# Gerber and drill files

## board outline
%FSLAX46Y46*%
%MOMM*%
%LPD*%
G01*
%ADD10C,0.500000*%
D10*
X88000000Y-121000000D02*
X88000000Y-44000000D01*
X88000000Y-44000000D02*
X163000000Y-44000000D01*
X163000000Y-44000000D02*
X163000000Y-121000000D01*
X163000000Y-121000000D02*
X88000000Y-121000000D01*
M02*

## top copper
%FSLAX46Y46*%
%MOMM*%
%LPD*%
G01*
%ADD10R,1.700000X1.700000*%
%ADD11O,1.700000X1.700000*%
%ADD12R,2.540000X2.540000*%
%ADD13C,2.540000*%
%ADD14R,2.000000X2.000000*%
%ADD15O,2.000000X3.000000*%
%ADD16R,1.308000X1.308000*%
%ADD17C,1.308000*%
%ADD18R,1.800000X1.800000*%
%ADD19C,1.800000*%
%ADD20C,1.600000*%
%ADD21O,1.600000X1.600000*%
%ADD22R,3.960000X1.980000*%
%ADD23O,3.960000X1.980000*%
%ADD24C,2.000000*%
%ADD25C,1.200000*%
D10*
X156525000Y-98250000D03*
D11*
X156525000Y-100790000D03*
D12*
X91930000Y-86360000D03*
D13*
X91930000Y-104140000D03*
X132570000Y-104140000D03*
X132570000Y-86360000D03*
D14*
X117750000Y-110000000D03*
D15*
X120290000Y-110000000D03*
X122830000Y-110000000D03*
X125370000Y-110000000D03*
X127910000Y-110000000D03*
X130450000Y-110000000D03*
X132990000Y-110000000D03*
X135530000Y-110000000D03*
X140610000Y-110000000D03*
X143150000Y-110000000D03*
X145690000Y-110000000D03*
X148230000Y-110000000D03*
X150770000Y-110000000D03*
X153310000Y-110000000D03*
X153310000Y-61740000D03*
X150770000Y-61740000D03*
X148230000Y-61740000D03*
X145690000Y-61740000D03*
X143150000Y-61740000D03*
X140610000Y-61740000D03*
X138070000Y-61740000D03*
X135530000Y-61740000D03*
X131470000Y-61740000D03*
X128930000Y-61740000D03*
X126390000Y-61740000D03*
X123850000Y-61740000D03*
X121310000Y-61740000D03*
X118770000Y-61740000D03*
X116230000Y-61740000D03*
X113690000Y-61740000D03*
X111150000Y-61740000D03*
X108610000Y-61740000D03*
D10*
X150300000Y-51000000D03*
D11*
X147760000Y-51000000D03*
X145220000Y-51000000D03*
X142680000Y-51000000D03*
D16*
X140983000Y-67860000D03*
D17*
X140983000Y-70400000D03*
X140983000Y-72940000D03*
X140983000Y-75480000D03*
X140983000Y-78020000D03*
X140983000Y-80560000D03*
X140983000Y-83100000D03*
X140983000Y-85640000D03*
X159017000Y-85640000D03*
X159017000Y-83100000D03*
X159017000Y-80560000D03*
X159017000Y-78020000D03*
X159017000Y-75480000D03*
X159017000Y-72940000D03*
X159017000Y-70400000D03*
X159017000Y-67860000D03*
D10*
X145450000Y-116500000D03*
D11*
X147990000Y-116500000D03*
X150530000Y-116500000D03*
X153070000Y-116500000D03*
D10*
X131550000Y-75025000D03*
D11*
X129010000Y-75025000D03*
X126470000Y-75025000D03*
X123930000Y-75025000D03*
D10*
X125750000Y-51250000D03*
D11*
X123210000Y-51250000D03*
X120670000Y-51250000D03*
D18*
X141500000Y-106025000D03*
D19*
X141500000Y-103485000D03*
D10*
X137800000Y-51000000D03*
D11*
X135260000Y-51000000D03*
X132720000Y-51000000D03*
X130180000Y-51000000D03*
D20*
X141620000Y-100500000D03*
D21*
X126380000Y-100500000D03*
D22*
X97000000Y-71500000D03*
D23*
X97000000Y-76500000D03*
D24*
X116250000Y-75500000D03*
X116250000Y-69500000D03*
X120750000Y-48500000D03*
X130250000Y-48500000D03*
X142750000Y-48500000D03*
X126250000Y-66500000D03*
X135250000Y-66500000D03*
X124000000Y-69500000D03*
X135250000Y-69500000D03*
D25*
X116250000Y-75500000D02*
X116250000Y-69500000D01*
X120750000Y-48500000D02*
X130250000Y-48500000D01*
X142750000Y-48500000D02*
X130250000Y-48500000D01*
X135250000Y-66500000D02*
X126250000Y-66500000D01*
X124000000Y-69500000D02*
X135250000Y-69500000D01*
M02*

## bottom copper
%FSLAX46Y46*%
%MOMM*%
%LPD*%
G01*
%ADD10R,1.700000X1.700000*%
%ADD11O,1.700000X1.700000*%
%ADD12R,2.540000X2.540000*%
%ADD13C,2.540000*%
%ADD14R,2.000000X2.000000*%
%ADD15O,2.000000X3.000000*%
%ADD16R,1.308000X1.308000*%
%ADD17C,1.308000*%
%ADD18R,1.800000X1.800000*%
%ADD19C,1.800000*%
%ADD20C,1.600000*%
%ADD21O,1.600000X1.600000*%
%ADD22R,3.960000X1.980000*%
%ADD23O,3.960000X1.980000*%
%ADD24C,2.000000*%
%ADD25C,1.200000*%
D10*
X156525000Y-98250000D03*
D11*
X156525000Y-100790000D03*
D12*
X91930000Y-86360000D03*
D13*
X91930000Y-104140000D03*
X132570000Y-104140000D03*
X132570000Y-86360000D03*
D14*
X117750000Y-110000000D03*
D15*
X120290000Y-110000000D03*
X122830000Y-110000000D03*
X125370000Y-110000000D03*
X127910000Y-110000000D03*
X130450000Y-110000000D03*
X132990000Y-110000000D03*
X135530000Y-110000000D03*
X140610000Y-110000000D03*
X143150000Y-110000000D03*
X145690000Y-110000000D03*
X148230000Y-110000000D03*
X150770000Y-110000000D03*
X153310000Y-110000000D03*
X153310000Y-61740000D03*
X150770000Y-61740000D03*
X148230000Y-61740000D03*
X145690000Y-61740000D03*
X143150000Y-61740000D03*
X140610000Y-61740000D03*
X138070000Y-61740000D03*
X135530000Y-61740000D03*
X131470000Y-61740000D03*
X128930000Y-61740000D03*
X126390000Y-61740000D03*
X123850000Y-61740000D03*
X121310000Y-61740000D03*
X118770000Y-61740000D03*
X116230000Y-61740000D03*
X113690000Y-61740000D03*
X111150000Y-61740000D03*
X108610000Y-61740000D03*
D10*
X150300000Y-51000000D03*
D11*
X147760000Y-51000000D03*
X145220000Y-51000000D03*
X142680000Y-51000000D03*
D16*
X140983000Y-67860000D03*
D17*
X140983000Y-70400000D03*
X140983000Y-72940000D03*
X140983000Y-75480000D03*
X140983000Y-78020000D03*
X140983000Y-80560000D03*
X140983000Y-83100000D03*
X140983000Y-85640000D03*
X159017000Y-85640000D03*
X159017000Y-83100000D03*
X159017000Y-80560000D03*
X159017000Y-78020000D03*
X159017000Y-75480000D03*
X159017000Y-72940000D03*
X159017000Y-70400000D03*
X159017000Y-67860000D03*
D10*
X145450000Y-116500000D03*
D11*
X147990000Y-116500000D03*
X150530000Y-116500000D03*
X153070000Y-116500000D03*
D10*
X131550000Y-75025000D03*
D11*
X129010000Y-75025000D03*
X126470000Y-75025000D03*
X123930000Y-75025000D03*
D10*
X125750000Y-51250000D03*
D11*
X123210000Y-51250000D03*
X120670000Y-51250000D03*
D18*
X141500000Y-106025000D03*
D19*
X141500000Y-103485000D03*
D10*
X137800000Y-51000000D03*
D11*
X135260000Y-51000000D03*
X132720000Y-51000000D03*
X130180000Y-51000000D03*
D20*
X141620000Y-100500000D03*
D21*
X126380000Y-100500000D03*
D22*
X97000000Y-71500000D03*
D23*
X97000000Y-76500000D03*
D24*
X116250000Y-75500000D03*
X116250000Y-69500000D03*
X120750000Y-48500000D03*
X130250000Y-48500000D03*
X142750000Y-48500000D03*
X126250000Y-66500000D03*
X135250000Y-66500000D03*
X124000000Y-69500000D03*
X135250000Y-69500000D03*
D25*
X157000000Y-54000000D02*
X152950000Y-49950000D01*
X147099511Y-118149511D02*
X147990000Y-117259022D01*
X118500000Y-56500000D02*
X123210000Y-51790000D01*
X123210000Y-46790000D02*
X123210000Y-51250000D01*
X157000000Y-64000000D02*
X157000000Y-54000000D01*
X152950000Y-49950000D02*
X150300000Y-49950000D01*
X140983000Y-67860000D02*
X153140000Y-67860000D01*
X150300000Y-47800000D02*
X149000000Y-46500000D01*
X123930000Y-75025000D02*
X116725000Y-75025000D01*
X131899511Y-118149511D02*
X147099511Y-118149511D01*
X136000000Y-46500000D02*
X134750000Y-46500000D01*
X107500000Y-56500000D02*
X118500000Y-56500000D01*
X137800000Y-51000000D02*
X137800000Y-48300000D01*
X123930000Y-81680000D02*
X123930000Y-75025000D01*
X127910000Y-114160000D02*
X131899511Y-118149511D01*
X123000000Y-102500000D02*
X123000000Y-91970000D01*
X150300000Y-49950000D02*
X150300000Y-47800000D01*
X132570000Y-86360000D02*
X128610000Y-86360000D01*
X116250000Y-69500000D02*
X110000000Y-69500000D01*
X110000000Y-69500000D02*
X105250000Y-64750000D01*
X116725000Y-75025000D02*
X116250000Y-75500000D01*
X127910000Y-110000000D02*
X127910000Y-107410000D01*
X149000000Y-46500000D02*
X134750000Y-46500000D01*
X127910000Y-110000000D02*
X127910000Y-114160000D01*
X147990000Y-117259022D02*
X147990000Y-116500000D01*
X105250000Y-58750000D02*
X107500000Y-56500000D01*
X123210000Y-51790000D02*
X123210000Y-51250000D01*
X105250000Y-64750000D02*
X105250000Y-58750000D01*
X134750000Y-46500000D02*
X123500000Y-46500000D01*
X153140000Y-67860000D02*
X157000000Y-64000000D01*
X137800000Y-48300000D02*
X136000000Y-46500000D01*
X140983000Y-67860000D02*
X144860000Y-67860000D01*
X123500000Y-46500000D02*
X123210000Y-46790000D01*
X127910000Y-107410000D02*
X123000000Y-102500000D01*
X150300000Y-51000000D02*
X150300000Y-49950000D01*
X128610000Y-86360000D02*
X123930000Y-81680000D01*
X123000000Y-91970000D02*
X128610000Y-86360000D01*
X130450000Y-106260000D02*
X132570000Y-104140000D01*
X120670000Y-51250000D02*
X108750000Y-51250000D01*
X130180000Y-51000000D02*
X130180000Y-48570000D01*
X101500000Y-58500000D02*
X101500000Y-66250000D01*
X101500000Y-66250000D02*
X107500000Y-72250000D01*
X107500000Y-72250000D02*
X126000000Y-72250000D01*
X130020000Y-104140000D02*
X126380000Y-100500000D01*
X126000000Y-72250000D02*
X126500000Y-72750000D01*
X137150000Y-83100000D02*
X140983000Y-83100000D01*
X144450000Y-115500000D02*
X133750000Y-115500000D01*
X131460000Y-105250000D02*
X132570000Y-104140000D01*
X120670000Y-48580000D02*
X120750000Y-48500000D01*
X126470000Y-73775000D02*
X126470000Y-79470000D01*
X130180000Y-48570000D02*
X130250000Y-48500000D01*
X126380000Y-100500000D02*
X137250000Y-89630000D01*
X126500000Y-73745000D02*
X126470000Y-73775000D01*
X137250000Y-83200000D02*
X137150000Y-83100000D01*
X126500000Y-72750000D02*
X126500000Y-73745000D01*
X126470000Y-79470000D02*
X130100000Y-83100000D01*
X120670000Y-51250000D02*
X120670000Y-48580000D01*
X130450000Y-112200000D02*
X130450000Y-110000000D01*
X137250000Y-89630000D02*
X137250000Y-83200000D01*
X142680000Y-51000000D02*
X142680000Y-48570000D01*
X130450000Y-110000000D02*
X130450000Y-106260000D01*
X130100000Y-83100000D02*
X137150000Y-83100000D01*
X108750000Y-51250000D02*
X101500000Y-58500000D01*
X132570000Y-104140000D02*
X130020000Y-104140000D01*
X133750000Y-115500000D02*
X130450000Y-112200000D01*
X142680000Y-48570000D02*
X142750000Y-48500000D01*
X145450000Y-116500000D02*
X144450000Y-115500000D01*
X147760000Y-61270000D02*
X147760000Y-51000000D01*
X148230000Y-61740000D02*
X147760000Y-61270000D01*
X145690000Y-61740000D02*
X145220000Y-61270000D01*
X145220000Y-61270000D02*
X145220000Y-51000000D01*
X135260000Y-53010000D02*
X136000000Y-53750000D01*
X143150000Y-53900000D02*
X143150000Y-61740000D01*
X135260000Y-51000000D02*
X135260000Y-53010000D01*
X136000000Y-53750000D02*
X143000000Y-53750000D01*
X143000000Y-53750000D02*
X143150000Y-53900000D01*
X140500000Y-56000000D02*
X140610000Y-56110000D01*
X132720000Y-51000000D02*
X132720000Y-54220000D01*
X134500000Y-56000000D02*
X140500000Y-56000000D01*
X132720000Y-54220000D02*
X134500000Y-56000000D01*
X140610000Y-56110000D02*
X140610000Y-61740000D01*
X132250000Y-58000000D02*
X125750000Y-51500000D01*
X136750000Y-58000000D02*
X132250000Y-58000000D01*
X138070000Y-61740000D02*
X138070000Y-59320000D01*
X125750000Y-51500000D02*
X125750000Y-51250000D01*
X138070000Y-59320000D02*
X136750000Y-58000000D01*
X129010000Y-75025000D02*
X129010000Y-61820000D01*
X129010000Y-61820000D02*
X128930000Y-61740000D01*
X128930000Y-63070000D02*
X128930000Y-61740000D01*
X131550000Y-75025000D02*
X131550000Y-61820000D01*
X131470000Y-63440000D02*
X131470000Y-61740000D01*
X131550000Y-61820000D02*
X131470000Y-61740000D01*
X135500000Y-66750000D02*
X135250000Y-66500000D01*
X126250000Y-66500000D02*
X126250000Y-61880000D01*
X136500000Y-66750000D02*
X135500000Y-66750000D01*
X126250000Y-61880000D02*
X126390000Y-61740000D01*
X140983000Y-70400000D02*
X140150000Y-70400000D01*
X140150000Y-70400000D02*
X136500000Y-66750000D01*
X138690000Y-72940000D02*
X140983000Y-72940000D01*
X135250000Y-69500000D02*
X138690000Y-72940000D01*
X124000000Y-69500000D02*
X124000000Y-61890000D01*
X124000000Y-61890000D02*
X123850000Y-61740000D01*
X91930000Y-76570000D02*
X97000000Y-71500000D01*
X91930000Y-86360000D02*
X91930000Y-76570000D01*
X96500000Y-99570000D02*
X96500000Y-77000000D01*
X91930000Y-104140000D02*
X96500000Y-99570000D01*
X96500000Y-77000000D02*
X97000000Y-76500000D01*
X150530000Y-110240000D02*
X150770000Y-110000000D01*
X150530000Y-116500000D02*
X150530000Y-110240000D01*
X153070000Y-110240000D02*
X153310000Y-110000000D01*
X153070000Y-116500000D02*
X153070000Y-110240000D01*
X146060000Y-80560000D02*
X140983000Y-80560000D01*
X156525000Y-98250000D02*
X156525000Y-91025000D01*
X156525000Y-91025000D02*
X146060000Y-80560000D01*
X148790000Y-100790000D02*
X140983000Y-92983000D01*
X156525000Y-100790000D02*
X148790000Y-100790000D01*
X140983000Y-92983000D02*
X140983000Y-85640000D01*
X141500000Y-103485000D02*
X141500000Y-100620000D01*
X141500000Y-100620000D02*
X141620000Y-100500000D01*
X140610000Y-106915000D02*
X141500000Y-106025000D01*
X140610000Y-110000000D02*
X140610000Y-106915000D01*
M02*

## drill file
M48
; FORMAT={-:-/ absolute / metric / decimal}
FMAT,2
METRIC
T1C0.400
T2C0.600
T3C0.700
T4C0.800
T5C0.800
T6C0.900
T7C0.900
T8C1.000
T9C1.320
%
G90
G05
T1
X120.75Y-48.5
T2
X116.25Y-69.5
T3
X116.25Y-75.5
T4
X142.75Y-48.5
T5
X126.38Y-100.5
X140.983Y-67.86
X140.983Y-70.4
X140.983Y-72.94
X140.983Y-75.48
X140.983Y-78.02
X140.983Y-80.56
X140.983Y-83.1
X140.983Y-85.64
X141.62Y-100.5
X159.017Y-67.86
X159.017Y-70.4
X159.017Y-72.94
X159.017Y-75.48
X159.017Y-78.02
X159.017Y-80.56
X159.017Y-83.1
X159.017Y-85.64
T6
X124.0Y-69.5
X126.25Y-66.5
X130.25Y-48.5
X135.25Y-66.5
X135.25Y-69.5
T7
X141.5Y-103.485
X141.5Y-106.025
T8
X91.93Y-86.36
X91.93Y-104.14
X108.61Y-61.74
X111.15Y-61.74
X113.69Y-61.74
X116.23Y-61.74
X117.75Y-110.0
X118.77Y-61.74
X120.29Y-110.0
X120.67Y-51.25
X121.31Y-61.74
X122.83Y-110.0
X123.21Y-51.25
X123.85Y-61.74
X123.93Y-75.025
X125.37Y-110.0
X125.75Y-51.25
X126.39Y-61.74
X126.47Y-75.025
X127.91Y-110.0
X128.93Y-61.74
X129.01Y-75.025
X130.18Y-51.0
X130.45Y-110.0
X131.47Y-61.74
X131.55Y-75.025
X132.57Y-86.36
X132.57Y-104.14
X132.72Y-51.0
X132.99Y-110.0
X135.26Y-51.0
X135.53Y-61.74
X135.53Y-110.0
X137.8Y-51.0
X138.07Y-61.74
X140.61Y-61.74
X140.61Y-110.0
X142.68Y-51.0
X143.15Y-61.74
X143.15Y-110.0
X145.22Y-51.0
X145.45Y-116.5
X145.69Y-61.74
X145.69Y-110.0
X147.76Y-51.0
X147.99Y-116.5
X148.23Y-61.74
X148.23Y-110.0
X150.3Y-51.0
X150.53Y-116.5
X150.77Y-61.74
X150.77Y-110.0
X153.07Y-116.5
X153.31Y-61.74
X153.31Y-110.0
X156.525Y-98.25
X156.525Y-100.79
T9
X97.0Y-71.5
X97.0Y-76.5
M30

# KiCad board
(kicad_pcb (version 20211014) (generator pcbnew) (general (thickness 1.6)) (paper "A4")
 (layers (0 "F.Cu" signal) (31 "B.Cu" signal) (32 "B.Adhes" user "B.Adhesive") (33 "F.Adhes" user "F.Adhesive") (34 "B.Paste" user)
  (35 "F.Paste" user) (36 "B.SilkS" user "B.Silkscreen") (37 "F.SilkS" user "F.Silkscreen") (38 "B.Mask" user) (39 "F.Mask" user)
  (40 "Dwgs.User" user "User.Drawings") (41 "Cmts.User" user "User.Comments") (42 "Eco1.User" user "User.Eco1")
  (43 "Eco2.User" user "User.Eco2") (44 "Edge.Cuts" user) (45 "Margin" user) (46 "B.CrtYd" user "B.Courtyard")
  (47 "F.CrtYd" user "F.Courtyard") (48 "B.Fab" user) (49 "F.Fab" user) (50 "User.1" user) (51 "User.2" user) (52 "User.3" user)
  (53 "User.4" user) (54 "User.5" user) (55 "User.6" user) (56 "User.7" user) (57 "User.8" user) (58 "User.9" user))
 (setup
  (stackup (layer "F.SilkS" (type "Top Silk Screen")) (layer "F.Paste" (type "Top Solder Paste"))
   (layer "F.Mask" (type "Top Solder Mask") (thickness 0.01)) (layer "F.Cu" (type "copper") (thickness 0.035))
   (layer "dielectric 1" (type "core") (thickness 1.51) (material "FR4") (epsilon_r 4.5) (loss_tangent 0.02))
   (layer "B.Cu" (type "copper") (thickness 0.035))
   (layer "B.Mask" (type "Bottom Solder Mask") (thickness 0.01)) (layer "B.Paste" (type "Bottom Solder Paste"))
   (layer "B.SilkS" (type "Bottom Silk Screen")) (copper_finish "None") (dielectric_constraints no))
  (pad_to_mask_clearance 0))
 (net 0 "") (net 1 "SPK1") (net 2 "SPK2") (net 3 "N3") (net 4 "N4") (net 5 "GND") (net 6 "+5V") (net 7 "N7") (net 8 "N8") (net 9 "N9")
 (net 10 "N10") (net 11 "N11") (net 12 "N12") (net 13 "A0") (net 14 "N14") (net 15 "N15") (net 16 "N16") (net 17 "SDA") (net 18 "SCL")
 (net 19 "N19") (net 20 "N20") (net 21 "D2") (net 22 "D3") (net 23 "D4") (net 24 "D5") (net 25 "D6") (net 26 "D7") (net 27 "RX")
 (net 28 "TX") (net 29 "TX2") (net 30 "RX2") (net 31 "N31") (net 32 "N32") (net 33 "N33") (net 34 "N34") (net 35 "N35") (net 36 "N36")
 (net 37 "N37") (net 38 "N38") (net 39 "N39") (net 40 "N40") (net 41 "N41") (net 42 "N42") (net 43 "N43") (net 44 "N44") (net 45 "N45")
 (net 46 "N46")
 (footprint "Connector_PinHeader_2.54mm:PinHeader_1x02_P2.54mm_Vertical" (layer "F.Cu") (at 156.525 98.25)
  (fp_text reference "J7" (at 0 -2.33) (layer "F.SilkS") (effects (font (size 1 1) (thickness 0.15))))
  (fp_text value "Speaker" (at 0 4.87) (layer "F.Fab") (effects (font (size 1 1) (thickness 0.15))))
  (pad "1" thru_hole rect (at 0 0) (size 1.7 1.7) (drill 1) (layers *.Cu *.Mask) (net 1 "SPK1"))
  (pad "2" thru_hole oval (at 0 2.54) (size 1.7 1.7) (drill 1) (layers *.Cu *.Mask) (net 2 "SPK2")))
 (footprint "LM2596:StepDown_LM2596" (layer "F.Cu") (at 91.93 86.36)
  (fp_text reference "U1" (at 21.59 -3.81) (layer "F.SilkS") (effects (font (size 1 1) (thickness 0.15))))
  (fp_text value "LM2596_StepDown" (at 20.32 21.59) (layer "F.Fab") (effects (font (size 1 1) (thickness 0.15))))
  (pad "1" thru_hole rect (at 0 0) (size 2.54 2.54) (drill 1) (layers *.Cu *.Mask) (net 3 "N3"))
  (pad "2" thru_hole circle (at 0 17.78) (size 2.54 2.54) (drill 1) (layers *.Cu *.Mask) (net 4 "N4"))
  (pad "3" thru_hole circle (at 40.64 17.78) (size 2.54 2.54) (drill 1) (layers *.Cu *.Mask) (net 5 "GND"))
  (pad "4" thru_hole circle (at 40.64 0) (size 2.54 2.54) (drill 1) (layers *.Cu *.Mask) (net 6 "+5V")))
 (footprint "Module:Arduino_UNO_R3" (layer "F.Cu") (at 117.75 64)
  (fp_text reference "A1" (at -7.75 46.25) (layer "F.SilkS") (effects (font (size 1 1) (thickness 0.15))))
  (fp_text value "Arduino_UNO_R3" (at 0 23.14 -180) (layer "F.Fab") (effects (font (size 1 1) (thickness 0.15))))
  (pad "1" thru_hole rect (at 0 46 90) (size 2 2) (drill 1) (layers *.Cu *.Mask) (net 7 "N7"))
  (pad "2" thru_hole oval (at 2.54 46 90) (size 3 2) (drill 1) (layers *.Cu *.Mask) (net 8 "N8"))
  (pad "3" thru_hole oval (at 5.08 46 90) (size 3 2) (drill 1) (layers *.Cu *.Mask) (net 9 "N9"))
  (pad "4" thru_hole oval (at 7.62 46 90) (size 3 2) (drill 1) (layers *.Cu *.Mask) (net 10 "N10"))
  (pad "5" thru_hole oval (at 10.16 46 90) (size 3 2) (drill 1) (layers *.Cu *.Mask) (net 6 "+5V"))
  (pad "6" thru_hole oval (at 12.7 46 90) (size 3 2) (drill 1) (layers *.Cu *.Mask) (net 5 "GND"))
  (pad "7" thru_hole oval (at 15.24 46 90) (size 3 2) (drill 1) (layers *.Cu *.Mask) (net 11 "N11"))
  (pad "8" thru_hole oval (at 17.78 46 90) (size 3 2) (drill 1) (layers *.Cu *.Mask) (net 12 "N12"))
  (pad "9" thru_hole oval (at 22.86 46 90) (size 3 2) (drill 1) (layers *.Cu *.Mask) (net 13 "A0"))
  (pad "10" thru_hole oval (at 25.4 46 90) (size 3 2) (drill 1) (layers *.Cu *.Mask) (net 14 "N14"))
  (pad "11" thru_hole oval (at 27.94 46 90) (size 3 2) (drill 1) (layers *.Cu *.Mask) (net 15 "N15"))
  (pad "12" thru_hole oval (at 30.48 46 90) (size 3 2) (drill 1) (layers *.Cu *.Mask) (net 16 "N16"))
  (pad "13" thru_hole oval (at 33.02 46 90) (size 3 2) (drill 1) (layers *.Cu *.Mask) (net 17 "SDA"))
  (pad "14" thru_hole oval (at 35.56 46 90) (size 3 2) (drill 1) (layers *.Cu *.Mask) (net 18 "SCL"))
  (pad "15" thru_hole oval (at 35.56 -2.26 90) (size 3 2) (drill 1) (layers *.Cu *.Mask) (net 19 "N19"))
  (pad "16" thru_hole oval (at 33.02 -2.26 90) (size 3 2) (drill 1) (layers *.Cu *.Mask) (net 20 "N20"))
  (pad "17" thru_hole oval (at 30.48 -2.26 90) (size 3 2) (drill 1) (layers *.Cu *.Mask) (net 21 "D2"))
  (pad "18" thru_hole oval (at 27.94 -2.26 90) (size 3 2) (drill 1) (layers *.Cu *.Mask) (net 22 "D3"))
  (pad "19" thru_hole oval (at 25.4 -2.26 90) (size 3 2) (drill 1) (layers *.Cu *.Mask) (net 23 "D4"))
  (pad "20" thru_hole oval (at 22.86 -2.26 90) (size 3 2) (drill 1) (layers *.Cu *.Mask) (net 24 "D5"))
  (pad "21" thru_hole oval (at 20.32 -2.26 90) (size 3 2) (drill 1) (layers *.Cu *.Mask) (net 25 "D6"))
  (pad "22" thru_hole oval (at 17.78 -2.26 90) (size 3 2) (drill 1) (layers *.Cu *.Mask) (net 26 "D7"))
  (pad "23" thru_hole oval (at 13.72 -2.26 90) (size 3 2) (drill 1) (layers *.Cu *.Mask) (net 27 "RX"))
  (pad "24" thru_hole oval (at 11.18 -2.26 90) (size 3 2) (drill 1) (layers *.Cu *.Mask) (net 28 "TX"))
  (pad "25" thru_hole oval (at 8.64 -2.26 90) (size 3 2) (drill 1) (layers *.Cu *.Mask) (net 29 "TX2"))
  (pad "26" thru_hole oval (at 6.1 -2.26 90) (size 3 2) (drill 1) (layers *.Cu *.Mask) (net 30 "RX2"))
  (pad "27" thru_hole oval (at 3.56 -2.26 90) (size 3 2) (drill 1) (layers *.Cu *.Mask) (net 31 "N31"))
  (pad "28" thru_hole oval (at 1.02 -2.26 90) (size 3 2) (drill 1) (layers *.Cu *.Mask) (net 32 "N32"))
  (pad "29" thru_hole oval (at -1.52 -2.26 90) (size 3 2) (drill 1) (layers *.Cu *.Mask) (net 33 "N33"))
  (pad "30" thru_hole oval (at -4.06 -2.26 90) (size 3 2) (drill 1) (layers *.Cu *.Mask) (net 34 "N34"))
  (pad "31" thru_hole oval (at -6.6 -2.26 90) (size 3 2) (drill 1) (layers *.Cu *.Mask) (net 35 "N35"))
  (pad "32" thru_hole oval (at -9.14 -2.26 90) (size 3 2) (drill 1) (layers *.Cu *.Mask) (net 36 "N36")))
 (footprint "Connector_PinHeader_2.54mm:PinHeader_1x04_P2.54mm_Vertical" (layer "F.Cu") (at 150.3 51 -90)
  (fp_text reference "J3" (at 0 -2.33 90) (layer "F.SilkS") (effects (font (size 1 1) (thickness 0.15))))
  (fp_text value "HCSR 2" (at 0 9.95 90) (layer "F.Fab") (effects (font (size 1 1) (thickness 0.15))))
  (pad "1" thru_hole rect (at 0 0 270) (size 1.7 1.7) (drill 1) (layers *.Cu *.Mask) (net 6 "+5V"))
  (pad "2" thru_hole oval (at 0 2.54 270) (size 1.7 1.7) (drill 1) (layers *.Cu *.Mask) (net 21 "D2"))
  (pad "3" thru_hole oval (at 0 5.08 270) (size 1.7 1.7) (drill 1) (layers *.Cu *.Mask) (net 22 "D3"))
  (pad "4" thru_hole oval (at 0 7.62 270) (size 1.7 1.7) (drill 1) (layers *.Cu *.Mask) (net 5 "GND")))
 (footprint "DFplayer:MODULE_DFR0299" (layer "F.Cu") (at 150 76.75)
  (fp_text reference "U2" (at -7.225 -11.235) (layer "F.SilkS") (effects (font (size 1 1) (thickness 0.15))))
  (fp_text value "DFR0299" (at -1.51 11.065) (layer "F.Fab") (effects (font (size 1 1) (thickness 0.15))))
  (pad "1" thru_hole rect (at -9.017 -8.89) (size 1.308 1.308) (drill 0.8) (layers *.Cu *.Mask) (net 6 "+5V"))
  (pad "2" thru_hole circle (at -9.017 -6.35) (size 1.308 1.308) (drill 0.8) (layers *.Cu *.Mask) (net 29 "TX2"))
  (pad "3" thru_hole circle (at -9.017 -3.81) (size 1.308 1.308) (drill 0.8) (layers *.Cu *.Mask) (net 30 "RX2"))
  (pad "4" thru_hole circle (at -9.017 -1.27) (size 1.308 1.308) (drill 0.8) (layers *.Cu *.Mask) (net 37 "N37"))
  (pad "5" thru_hole circle (at -9.017 1.27) (size 1.308 1.308) (drill 0.8) (layers *.Cu *.Mask) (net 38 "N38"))
  (pad "6" thru_hole circle (at -9.017 3.81) (size 1.308 1.308) (drill 0.8) (layers *.Cu *.Mask) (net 1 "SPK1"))
  (pad "7" thru_hole circle (at -9.017 6.35) (size 1.308 1.308) (drill 0.8) (layers *.Cu *.Mask) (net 5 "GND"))
  (pad "8" thru_hole circle (at -9.017 8.89) (size 1.308 1.308) (drill 0.8) (layers *.Cu *.Mask) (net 2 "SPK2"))
  (pad "9" thru_hole circle (at 9.017 8.89) (size 1.308 1.308) (drill 0.8) (layers *.Cu *.Mask) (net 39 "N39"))
  (pad "10" thru_hole circle (at 9.017 6.35) (size 1.308 1.308) (drill 0.8) (layers *.Cu *.Mask) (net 5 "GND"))
  (pad "11" thru_hole circle (at 9.017 3.81) (size 1.308 1.308) (drill 0.8) (layers *.Cu *.Mask) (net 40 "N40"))
  (pad "12" thru_hole circle (at 9.017 1.27) (size 1.308 1.308) (drill 0.8) (layers *.Cu *.Mask) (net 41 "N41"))
  (pad "13" thru_hole circle (at 9.017 -1.27) (size 1.308 1.308) (drill 0.8) (layers *.Cu *.Mask) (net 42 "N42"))
  (pad "14" thru_hole circle (at 9.017 -3.81) (size 1.308 1.308) (drill 0.8) (layers *.Cu *.Mask) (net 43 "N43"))
  (pad "15" thru_hole circle (at 9.017 -6.35) (size 1.308 1.308) (drill 0.8) (layers *.Cu *.Mask) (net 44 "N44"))
  (pad "16" thru_hole circle (at 9.017 -8.89) (size 1.308 1.308) (drill 0.8) (layers *.Cu *.Mask) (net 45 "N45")))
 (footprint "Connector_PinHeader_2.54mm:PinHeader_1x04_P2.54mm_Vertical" (layer "F.Cu") (at 145.45 116.5 90)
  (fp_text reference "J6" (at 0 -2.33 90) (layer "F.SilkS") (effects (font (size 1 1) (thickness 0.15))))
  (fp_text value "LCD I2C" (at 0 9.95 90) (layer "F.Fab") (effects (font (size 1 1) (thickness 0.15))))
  (pad "1" thru_hole rect (at 0 0 90) (size 1.7 1.7) (drill 1) (layers *.Cu *.Mask) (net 5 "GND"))
  (pad "2" thru_hole oval (at 0 2.54 90) (size 1.7 1.7) (drill 1) (layers *.Cu *.Mask) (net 6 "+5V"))
  (pad "3" thru_hole oval (at 0 5.08 90) (size 1.7 1.7) (drill 1) (layers *.Cu *.Mask) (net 17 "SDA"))
  (pad "4" thru_hole oval (at 0 7.62 90) (size 1.7 1.7) (drill 1) (layers *.Cu *.Mask) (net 18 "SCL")))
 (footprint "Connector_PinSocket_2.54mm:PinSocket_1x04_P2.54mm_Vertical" (layer "F.Cu") (at 131.55 75.025 -90)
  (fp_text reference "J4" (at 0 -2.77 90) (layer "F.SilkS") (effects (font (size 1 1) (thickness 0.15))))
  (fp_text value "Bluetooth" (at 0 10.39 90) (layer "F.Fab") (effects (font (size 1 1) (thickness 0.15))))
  (pad "1" thru_hole rect (at 0 0 270) (size 1.7 1.7) (drill 1) (layers *.Cu *.Mask) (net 27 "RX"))
  (pad "2" thru_hole oval (at 0 2.54 270) (size 1.7 1.7) (drill 1) (layers *.Cu *.Mask) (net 28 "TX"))
  (pad "3" thru_hole oval (at 0 5.08 270) (size 1.7 1.7) (drill 1) (layers *.Cu *.Mask) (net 5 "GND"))
  (pad "4" thru_hole oval (at 0 7.62 270) (size 1.7 1.7) (drill 1) (layers *.Cu *.Mask) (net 6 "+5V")))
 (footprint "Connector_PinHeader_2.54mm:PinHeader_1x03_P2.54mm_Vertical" (layer "F.Cu") (at 125.75 51.25 -90)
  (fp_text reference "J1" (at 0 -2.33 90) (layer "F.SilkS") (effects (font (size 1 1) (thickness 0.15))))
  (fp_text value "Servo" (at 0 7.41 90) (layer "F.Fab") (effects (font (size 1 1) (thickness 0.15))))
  (pad "1" thru_hole rect (at 0 0 270) (size 1.7 1.7) (drill 1) (layers *.Cu *.Mask) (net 25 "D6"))
  (pad "2" thru_hole oval (at 0 2.54 270) (size 1.7 1.7) (drill 1) (layers *.Cu *.Mask) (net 6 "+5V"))
  (pad "3" thru_hole oval (at 0 5.08 270) (size 1.7 1.7) (drill 1) (layers *.Cu *.Mask) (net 5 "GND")))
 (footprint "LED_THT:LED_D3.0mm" (layer "F.Cu") (at 141.5 106.025 90)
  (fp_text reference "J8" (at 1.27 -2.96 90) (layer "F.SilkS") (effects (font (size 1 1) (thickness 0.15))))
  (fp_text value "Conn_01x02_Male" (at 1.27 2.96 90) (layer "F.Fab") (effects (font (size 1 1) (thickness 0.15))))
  (pad "1" thru_hole rect (at 0 0 90) (size 1.8 1.8) (drill 0.9) (layers *.Cu *.Mask) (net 13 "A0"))
  (pad "2" thru_hole circle (at 2.54 0 90) (size 1.8 1.8) (drill 0.9) (layers *.Cu *.Mask) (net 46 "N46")))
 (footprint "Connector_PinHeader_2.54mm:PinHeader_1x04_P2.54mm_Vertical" (layer "F.Cu") (at 137.8 51 -90)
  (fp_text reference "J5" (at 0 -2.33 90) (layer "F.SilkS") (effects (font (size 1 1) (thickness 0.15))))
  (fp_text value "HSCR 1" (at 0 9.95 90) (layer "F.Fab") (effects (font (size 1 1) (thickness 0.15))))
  (pad "1" thru_hole rect (at 0 0 270) (size 1.7 1.7) (drill 1) (layers *.Cu *.Mask) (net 6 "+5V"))
  (pad "2" thru_hole oval (at 0 2.54 270) (size 1.7 1.7) (drill 1) (layers *.Cu *.Mask) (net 23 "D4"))
  (pad "3" thru_hole oval (at 0 5.08 270) (size 1.7 1.7) (drill 1) (layers *.Cu *.Mask) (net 24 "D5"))
  (pad "4" thru_hole oval (at 0 7.62 270) (size 1.7 1.7) (drill 1) (layers *.Cu *.Mask) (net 5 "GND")))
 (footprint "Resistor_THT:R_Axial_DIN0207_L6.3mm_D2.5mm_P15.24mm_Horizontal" (layer "F.Cu") (at 141.62 100.5 180)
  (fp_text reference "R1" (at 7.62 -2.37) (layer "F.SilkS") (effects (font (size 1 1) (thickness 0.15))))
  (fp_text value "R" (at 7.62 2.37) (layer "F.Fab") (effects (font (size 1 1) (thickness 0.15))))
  (pad "1" thru_hole circle (at 0 0 180) (size 1.6 1.6) (drill 0.8) (layers *.Cu *.Mask) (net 46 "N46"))
  (pad "2" thru_hole oval (at 15.24 0 180) (size 1.6 1.6) (drill 0.8) (layers *.Cu *.Mask) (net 5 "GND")))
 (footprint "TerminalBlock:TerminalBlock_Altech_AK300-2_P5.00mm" (layer "F.Cu") (at 97 71.5 -90)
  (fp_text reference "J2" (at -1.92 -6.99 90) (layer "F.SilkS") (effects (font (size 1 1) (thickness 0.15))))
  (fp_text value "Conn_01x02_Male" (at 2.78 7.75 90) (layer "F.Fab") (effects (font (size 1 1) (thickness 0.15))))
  (pad "1" thru_hole rect (at 0 0 270) (size 1.98 3.96) (drill 1.32) (layers *.Cu *.Mask) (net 3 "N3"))
  (pad "2" thru_hole oval (at 5 0 270) (size 1.98 3.96) (drill 1.32) (layers *.Cu *.Mask) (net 4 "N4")))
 (gr_line (start 88 121) (end 88 44) (layer "Edge.Cuts") (width 0.5))
 (gr_line (start 88 44) (end 163 44) (layer "Edge.Cuts") (width 0.5))
 (gr_line (start 163 44) (end 163 121) (layer "Edge.Cuts") (width 0.5))
 (gr_line (start 163 121) (end 88 121) (layer "Edge.Cuts") (width 0.5))
 (segment (start 116.25 75.5) (end 116.25 69.5) (width 1.2) (layer "F.Cu") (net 6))
 (via (at 116.25 75.5) (size 2) (drill 0.7) (layers "F.Cu" "B.Cu") (free) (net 6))
 (via (at 116.25 69.5) (size 2) (drill 0.6) (layers "F.Cu" "B.Cu") (free) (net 6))
 (segment (start 157 54) (end 152.95 49.95) (width 1.2) (layer "B.Cu") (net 6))
 (segment (start 147.099511 118.149511) (end 147.99 117.259022) (width 1.2) (layer "B.Cu") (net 6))
 (segment (start 118.5 56.5) (end 123.21 51.79) (width 1.2) (layer "B.Cu") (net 6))
 (segment (start 123.21 46.79) (end 123.21 51.25) (width 1.2) (layer "B.Cu") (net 6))
 (segment (start 157 64) (end 157 54) (width 1.2) (layer "B.Cu") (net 6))
 (segment (start 152.95 49.95) (end 150.3 49.95) (width 1.2) (layer "B.Cu") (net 6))
 (segment (start 140.983 67.86) (end 153.14 67.86) (width 1.2) (layer "B.Cu") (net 6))
 (segment (start 150.3 47.8) (end 149 46.5) (width 1.2) (layer "B.Cu") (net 6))
 (segment (start 123.93 75.025) (end 116.725 75.025) (width 1.2) (layer "B.Cu") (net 6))
 (segment (start 131.899511 118.149511) (end 147.099511 118.149511) (width 1.2) (layer "B.Cu") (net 6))
 (segment (start 136 46.5) (end 134.75 46.5) (width 1.2) (layer "B.Cu") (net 6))
 (segment (start 107.5 56.5) (end 118.5 56.5) (width 1.2) (layer "B.Cu") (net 6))
 (segment (start 137.8 51) (end 137.8 48.3) (width 1.2) (layer "B.Cu") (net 6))
 (segment (start 123.93 81.68) (end 123.93 75.025) (width 1.2) (layer "B.Cu") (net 6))
 (segment (start 127.91 114.16) (end 131.899511 118.149511) (width 1.2) (layer "B.Cu") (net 6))
 (segment (start 123 102.5) (end 123 91.97) (width 1.2) (layer "B.Cu") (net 6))
 (segment (start 150.3 49.95) (end 150.3 47.8) (width 1.2) (layer "B.Cu") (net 6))
 (segment (start 132.57 86.36) (end 128.61 86.36) (width 1.2) (layer "B.Cu") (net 6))
 (segment (start 116.25 69.5) (end 110 69.5) (width 1.2) (layer "B.Cu") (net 6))
 (segment (start 110 69.5) (end 105.25 64.75) (width 1.2) (layer "B.Cu") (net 6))
 (segment (start 116.725 75.025) (end 116.25 75.5) (width 1.2) (layer "B.Cu") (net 6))
 (segment (start 127.91 110) (end 127.91 107.41) (width 1.2) (layer "B.Cu") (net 6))
 (segment (start 149 46.5) (end 134.75 46.5) (width 1.2) (layer "B.Cu") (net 6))
 (segment (start 127.91 110) (end 127.91 114.16) (width 1.2) (layer "B.Cu") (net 6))
 (segment (start 147.99 117.259022) (end 147.99 116.5) (width 1.2) (layer "B.Cu") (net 6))
 (segment (start 105.25 58.75) (end 107.5 56.5) (width 1.2) (layer "B.Cu") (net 6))
 (segment (start 123.21 51.79) (end 123.21 51.25) (width 1.2) (layer "B.Cu") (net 6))
 (segment (start 105.25 64.75) (end 105.25 58.75) (width 1.2) (layer "B.Cu") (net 6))
 (segment (start 134.75 46.5) (end 123.5 46.5) (width 1.2) (layer "B.Cu") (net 6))
 (segment (start 153.14 67.86) (end 157 64) (width 1.2) (layer "B.Cu") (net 6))
 (segment (start 137.8 48.3) (end 136 46.5) (width 1.2) (layer "B.Cu") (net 6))
 (segment (start 140.983 67.86) (end 144.86 67.86) (width 1.2) (layer "B.Cu") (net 6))
 (segment (start 123.5 46.5) (end 123.21 46.79) (width 1.2) (layer "B.Cu") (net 6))
 (segment (start 127.91 107.41) (end 123 102.5) (width 1.2) (layer "B.Cu") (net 6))
 (segment (start 150.3 51) (end 150.3 49.95) (width 1.2) (layer "B.Cu") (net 6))
 (segment (start 128.61 86.36) (end 123.93 81.68) (width 1.2) (layer "B.Cu") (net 6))
 (segment (start 123 91.97) (end 128.61 86.36) (width 1.2) (layer "B.Cu") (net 6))
 (segment (start 120.75 48.5) (end 130.25 48.5) (width 1.2) (layer "F.Cu") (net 5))
 (segment (start 142.75 48.5) (end 130.25 48.5) (width 1.2) (layer "F.Cu") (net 5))
 (via (at 120.75 48.5) (size 2) (drill 0.4) (layers "F.Cu" "B.Cu") (free) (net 5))
 (via (at 130.25 48.5) (size 2) (drill 0.9) (layers "F.Cu" "B.Cu") (free) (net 5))
 (via (at 142.75 48.5) (size 2) (drill 0.8) (layers "F.Cu" "B.Cu") (free) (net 5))
 (segment (start 130.45 106.26) (end 132.57 104.14) (width 1.2) (layer "B.Cu") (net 5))
 (segment (start 120.67 51.25) (end 108.75 51.25) (width 1.2) (layer "B.Cu") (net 5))
 (segment (start 130.18 51) (end 130.18 48.57) (width 1.2) (layer "B.Cu") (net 5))
 (segment (start 101.5 58.5) (end 101.5 66.25) (width 1.2) (layer "B.Cu") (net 5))
 (segment (start 101.5 66.25) (end 107.5 72.25) (width 1.2) (layer "B.Cu") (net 5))
 (segment (start 107.5 72.25) (end 126 72.25) (width 1.2) (layer "B.Cu") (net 5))
 (segment (start 130.02 104.14) (end 126.38 100.5) (width 1.2) (layer "B.Cu") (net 5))
 (segment (start 126 72.25) (end 126.5 72.75) (width 1.2) (layer "B.Cu") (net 5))
 (segment (start 137.15 83.1) (end 140.983 83.1) (width 1.2) (layer "B.Cu") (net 5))
 (segment (start 144.45 115.5) (end 133.75 115.5) (width 1.2) (layer "B.Cu") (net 5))
 (segment (start 131.46 105.25) (end 132.57 104.14) (width 1.2) (layer "B.Cu") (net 5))
 (segment (start 120.67 48.58) (end 120.75 48.5) (width 1.2) (layer "B.Cu") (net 5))
 (segment (start 126.47 73.775) (end 126.47 79.47) (width 1.2) (layer "B.Cu") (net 5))
 (segment (start 130.18 48.57) (end 130.25 48.5) (width 1.2) (layer "B.Cu") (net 5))
 (segment (start 126.38 100.5) (end 137.25 89.63) (width 1.2) (layer "B.Cu") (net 5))
 (segment (start 126.5 73.745) (end 126.47 73.775) (width 1.2) (layer "B.Cu") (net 5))
 (segment (start 137.25 83.2) (end 137.15 83.1) (width 1.2) (layer "B.Cu") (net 5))
 (segment (start 126.5 72.75) (end 126.5 73.745) (width 1.2) (layer "B.Cu") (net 5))
 (segment (start 126.47 79.47) (end 130.1 83.1) (width 1.2) (layer "B.Cu") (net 5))
 (segment (start 120.67 51.25) (end 120.67 48.58) (width 1.2) (layer "B.Cu") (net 5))
 (segment (start 130.45 112.2) (end 130.45 110) (width 1.2) (layer "B.Cu") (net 5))
 (segment (start 137.25 89.63) (end 137.25 83.2) (width 1.2) (layer "B.Cu") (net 5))
 (segment (start 142.68 51) (end 142.68 48.57) (width 1.2) (layer "B.Cu") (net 5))
 (segment (start 130.45 110) (end 130.45 106.26) (width 1.2) (layer "B.Cu") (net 5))
 (segment (start 130.1 83.1) (end 137.15 83.1) (width 1.2) (layer "B.Cu") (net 5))
 (segment (start 108.75 51.25) (end 101.5 58.5) (width 1.2) (layer "B.Cu") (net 5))
 (segment (start 132.57 104.14) (end 130.02 104.14) (width 1.2) (layer "B.Cu") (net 5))
 (segment (start 133.75 115.5) (end 130.45 112.2) (width 1.2) (layer "B.Cu") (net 5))
 (segment (start 142.68 48.57) (end 142.75 48.5) (width 1.2) (layer "B.Cu") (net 5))
 (segment (start 145.45 116.5) (end 144.45 115.5) (width 1.2) (layer "B.Cu") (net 5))
 (segment (start 147.76 61.27) (end 147.76 51) (width 1.2) (layer "B.Cu") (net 21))
 (segment (start 148.23 61.74) (end 147.76 61.27) (width 1.2) (layer "B.Cu") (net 21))
 (segment (start 145.69 61.74) (end 145.22 61.27) (width 1.2) (layer "B.Cu") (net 22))
 (segment (start 145.22 61.27) (end 145.22 51) (width 1.2) (layer "B.Cu") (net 22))
 (segment (start 135.26 53.01) (end 136 53.75) (width 1.2) (layer "B.Cu") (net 23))
 (segment (start 143.15 53.9) (end 143.15 61.74) (width 1.2) (layer "B.Cu") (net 23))
 (segment (start 135.26 51) (end 135.26 53.01) (width 1.2) (layer "B.Cu") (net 23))
 (segment (start 136 53.75) (end 143 53.75) (width 1.2) (layer "B.Cu") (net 23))
 (segment (start 143 53.75) (end 143.15 53.9) (width 1.2) (layer "B.Cu") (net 23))
 (segment (start 140.5 56) (end 140.61 56.11) (width 1.2) (layer "B.Cu") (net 24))
 (segment (start 132.72 51) (end 132.72 54.22) (width 1.2) (layer "B.Cu") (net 24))
 (segment (start 134.5 56) (end 140.5 56) (width 1.2) (layer "B.Cu") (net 24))
 (segment (start 132.72 54.22) (end 134.5 56) (width 1.2) (layer "B.Cu") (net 24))
 (segment (start 140.61 56.11) (end 140.61 61.74) (width 1.2) (layer "B.Cu") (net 24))
 (segment (start 132.25 58) (end 125.75 51.5) (width 1.2) (layer "B.Cu") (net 25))
 (segment (start 136.75 58) (end 132.25 58) (width 1.2) (layer "B.Cu") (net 25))
 (segment (start 138.07 61.74) (end 138.07 59.32) (width 1.2) (layer "B.Cu") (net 25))
 (segment (start 125.75 51.5) (end 125.75 51.25) (width 1.2) (layer "B.Cu") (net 25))
 (segment (start 138.07 59.32) (end 136.75 58) (width 1.2) (layer "B.Cu") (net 25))
 (segment (start 129.01 75.025) (end 129.01 61.82) (width 1.2) (layer "B.Cu") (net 28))
 (segment (start 129.01 61.82) (end 128.93 61.74) (width 1.2) (layer "B.Cu") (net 28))
 (segment (start 128.93 63.07) (end 128.93 61.74) (width 1.2) (layer "B.Cu") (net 28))
 (segment (start 131.55 75.025) (end 131.55 61.82) (width 1.2) (layer "B.Cu") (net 27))
 (segment (start 131.47 63.44) (end 131.47 61.74) (width 1.2) (layer "B.Cu") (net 27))
 (segment (start 131.55 61.82) (end 131.47 61.74) (width 1.2) (layer "B.Cu") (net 27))
 (segment (start 135.25 66.5) (end 126.25 66.5) (width 1.2) (layer "F.Cu") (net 29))
 (via (at 126.25 66.5) (size 2) (drill 0.9) (layers "F.Cu" "B.Cu") (free) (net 29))
 (via (at 135.25 66.5) (size 2) (drill 0.9) (layers "F.Cu" "B.Cu") (free) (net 29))
 (segment (start 135.5 66.75) (end 135.25 66.5) (width 1.2) (layer "B.Cu") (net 29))
 (segment (start 126.25 66.5) (end 126.25 61.88) (width 1.2) (layer "B.Cu") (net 29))
 (segment (start 136.5 66.75) (end 135.5 66.75) (width 1.2) (layer "B.Cu") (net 29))
 (segment (start 126.25 61.88) (end 126.39 61.74) (width 1.2) (layer "B.Cu") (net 29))
 (segment (start 140.983 70.4) (end 140.15 70.4) (width 1.2) (layer "B.Cu") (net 29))
 (segment (start 140.15 70.4) (end 136.5 66.75) (width 1.2) (layer "B.Cu") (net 29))
 (segment (start 124 69.5) (end 135.25 69.5) (width 1.2) (layer "F.Cu") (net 30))
 (via (at 124 69.5) (size 2) (drill 0.9) (layers "F.Cu" "B.Cu") (free) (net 30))
 (via (at 135.25 69.5) (size 2) (drill 0.9) (layers "F.Cu" "B.Cu") (free) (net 30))
 (segment (start 138.69 72.94) (end 140.983 72.94) (width 1.2) (layer "B.Cu") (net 30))
 (segment (start 135.25 69.5) (end 138.69 72.94) (width 1.2) (layer "B.Cu") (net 30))
 (segment (start 124 69.5) (end 124 61.89) (width 1.2) (layer "B.Cu") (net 30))
 (segment (start 124 61.89) (end 123.85 61.74) (width 1.2) (layer "B.Cu") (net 30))
 (segment (start 91.93 76.57) (end 97 71.5) (width 1.2) (layer "B.Cu") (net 3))
 (segment (start 91.93 86.36) (end 91.93 76.57) (width 1.2) (layer "B.Cu") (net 3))
 (segment (start 96.5 99.57) (end 96.5 77) (width 1.2) (layer "B.Cu") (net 4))
 (segment (start 91.93 104.14) (end 96.5 99.57) (width 1.2) (layer "B.Cu") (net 4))
 (segment (start 96.5 77) (end 97 76.5) (width 1.2) (layer "B.Cu") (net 4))
 (segment (start 150.53 110.24) (end 150.77 110) (width 1.2) (layer "B.Cu") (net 17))
 (segment (start 150.53 116.5) (end 150.53 110.24) (width 1.2) (layer "B.Cu") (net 17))
 (segment (start 153.07 110.24) (end 153.31 110) (width 1.2) (layer "B.Cu") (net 18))
 (segment (start 153.07 116.5) (end 153.07 110.24) (width 1.2) (layer "B.Cu") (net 18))
 (segment (start 146.06 80.56) (end 140.983 80.56) (width 1.2) (layer "B.Cu") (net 1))
 (segment (start 156.525 98.25) (end 156.525 91.025) (width 1.2) (layer "B.Cu") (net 1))
 (segment (start 156.525 91.025) (end 146.06 80.56) (width 1.2) (layer "B.Cu") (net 1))
 (segment (start 148.79 100.79) (end 140.983 92.983) (width 1.2) (layer "B.Cu") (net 2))
 (segment (start 156.525 100.79) (end 148.79 100.79) (width 1.2) (layer "B.Cu") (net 2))
 (segment (start 140.983 92.983) (end 140.983 85.64) (width 1.2) (layer "B.Cu") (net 2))
 (segment (start 141.5 103.485) (end 141.5 100.62) (width 1.2) (layer "B.Cu") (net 46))
 (segment (start 141.5 100.62) (end 141.62 100.5) (width 1.2) (layer "B.Cu") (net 46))
 (segment (start 140.61 106.915) (end 141.5 106.025) (width 1.2) (layer "B.Cu") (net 13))
 (segment (start 140.61 110) (end 140.61 106.915) (width 1.2) (layer "B.Cu") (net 13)))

